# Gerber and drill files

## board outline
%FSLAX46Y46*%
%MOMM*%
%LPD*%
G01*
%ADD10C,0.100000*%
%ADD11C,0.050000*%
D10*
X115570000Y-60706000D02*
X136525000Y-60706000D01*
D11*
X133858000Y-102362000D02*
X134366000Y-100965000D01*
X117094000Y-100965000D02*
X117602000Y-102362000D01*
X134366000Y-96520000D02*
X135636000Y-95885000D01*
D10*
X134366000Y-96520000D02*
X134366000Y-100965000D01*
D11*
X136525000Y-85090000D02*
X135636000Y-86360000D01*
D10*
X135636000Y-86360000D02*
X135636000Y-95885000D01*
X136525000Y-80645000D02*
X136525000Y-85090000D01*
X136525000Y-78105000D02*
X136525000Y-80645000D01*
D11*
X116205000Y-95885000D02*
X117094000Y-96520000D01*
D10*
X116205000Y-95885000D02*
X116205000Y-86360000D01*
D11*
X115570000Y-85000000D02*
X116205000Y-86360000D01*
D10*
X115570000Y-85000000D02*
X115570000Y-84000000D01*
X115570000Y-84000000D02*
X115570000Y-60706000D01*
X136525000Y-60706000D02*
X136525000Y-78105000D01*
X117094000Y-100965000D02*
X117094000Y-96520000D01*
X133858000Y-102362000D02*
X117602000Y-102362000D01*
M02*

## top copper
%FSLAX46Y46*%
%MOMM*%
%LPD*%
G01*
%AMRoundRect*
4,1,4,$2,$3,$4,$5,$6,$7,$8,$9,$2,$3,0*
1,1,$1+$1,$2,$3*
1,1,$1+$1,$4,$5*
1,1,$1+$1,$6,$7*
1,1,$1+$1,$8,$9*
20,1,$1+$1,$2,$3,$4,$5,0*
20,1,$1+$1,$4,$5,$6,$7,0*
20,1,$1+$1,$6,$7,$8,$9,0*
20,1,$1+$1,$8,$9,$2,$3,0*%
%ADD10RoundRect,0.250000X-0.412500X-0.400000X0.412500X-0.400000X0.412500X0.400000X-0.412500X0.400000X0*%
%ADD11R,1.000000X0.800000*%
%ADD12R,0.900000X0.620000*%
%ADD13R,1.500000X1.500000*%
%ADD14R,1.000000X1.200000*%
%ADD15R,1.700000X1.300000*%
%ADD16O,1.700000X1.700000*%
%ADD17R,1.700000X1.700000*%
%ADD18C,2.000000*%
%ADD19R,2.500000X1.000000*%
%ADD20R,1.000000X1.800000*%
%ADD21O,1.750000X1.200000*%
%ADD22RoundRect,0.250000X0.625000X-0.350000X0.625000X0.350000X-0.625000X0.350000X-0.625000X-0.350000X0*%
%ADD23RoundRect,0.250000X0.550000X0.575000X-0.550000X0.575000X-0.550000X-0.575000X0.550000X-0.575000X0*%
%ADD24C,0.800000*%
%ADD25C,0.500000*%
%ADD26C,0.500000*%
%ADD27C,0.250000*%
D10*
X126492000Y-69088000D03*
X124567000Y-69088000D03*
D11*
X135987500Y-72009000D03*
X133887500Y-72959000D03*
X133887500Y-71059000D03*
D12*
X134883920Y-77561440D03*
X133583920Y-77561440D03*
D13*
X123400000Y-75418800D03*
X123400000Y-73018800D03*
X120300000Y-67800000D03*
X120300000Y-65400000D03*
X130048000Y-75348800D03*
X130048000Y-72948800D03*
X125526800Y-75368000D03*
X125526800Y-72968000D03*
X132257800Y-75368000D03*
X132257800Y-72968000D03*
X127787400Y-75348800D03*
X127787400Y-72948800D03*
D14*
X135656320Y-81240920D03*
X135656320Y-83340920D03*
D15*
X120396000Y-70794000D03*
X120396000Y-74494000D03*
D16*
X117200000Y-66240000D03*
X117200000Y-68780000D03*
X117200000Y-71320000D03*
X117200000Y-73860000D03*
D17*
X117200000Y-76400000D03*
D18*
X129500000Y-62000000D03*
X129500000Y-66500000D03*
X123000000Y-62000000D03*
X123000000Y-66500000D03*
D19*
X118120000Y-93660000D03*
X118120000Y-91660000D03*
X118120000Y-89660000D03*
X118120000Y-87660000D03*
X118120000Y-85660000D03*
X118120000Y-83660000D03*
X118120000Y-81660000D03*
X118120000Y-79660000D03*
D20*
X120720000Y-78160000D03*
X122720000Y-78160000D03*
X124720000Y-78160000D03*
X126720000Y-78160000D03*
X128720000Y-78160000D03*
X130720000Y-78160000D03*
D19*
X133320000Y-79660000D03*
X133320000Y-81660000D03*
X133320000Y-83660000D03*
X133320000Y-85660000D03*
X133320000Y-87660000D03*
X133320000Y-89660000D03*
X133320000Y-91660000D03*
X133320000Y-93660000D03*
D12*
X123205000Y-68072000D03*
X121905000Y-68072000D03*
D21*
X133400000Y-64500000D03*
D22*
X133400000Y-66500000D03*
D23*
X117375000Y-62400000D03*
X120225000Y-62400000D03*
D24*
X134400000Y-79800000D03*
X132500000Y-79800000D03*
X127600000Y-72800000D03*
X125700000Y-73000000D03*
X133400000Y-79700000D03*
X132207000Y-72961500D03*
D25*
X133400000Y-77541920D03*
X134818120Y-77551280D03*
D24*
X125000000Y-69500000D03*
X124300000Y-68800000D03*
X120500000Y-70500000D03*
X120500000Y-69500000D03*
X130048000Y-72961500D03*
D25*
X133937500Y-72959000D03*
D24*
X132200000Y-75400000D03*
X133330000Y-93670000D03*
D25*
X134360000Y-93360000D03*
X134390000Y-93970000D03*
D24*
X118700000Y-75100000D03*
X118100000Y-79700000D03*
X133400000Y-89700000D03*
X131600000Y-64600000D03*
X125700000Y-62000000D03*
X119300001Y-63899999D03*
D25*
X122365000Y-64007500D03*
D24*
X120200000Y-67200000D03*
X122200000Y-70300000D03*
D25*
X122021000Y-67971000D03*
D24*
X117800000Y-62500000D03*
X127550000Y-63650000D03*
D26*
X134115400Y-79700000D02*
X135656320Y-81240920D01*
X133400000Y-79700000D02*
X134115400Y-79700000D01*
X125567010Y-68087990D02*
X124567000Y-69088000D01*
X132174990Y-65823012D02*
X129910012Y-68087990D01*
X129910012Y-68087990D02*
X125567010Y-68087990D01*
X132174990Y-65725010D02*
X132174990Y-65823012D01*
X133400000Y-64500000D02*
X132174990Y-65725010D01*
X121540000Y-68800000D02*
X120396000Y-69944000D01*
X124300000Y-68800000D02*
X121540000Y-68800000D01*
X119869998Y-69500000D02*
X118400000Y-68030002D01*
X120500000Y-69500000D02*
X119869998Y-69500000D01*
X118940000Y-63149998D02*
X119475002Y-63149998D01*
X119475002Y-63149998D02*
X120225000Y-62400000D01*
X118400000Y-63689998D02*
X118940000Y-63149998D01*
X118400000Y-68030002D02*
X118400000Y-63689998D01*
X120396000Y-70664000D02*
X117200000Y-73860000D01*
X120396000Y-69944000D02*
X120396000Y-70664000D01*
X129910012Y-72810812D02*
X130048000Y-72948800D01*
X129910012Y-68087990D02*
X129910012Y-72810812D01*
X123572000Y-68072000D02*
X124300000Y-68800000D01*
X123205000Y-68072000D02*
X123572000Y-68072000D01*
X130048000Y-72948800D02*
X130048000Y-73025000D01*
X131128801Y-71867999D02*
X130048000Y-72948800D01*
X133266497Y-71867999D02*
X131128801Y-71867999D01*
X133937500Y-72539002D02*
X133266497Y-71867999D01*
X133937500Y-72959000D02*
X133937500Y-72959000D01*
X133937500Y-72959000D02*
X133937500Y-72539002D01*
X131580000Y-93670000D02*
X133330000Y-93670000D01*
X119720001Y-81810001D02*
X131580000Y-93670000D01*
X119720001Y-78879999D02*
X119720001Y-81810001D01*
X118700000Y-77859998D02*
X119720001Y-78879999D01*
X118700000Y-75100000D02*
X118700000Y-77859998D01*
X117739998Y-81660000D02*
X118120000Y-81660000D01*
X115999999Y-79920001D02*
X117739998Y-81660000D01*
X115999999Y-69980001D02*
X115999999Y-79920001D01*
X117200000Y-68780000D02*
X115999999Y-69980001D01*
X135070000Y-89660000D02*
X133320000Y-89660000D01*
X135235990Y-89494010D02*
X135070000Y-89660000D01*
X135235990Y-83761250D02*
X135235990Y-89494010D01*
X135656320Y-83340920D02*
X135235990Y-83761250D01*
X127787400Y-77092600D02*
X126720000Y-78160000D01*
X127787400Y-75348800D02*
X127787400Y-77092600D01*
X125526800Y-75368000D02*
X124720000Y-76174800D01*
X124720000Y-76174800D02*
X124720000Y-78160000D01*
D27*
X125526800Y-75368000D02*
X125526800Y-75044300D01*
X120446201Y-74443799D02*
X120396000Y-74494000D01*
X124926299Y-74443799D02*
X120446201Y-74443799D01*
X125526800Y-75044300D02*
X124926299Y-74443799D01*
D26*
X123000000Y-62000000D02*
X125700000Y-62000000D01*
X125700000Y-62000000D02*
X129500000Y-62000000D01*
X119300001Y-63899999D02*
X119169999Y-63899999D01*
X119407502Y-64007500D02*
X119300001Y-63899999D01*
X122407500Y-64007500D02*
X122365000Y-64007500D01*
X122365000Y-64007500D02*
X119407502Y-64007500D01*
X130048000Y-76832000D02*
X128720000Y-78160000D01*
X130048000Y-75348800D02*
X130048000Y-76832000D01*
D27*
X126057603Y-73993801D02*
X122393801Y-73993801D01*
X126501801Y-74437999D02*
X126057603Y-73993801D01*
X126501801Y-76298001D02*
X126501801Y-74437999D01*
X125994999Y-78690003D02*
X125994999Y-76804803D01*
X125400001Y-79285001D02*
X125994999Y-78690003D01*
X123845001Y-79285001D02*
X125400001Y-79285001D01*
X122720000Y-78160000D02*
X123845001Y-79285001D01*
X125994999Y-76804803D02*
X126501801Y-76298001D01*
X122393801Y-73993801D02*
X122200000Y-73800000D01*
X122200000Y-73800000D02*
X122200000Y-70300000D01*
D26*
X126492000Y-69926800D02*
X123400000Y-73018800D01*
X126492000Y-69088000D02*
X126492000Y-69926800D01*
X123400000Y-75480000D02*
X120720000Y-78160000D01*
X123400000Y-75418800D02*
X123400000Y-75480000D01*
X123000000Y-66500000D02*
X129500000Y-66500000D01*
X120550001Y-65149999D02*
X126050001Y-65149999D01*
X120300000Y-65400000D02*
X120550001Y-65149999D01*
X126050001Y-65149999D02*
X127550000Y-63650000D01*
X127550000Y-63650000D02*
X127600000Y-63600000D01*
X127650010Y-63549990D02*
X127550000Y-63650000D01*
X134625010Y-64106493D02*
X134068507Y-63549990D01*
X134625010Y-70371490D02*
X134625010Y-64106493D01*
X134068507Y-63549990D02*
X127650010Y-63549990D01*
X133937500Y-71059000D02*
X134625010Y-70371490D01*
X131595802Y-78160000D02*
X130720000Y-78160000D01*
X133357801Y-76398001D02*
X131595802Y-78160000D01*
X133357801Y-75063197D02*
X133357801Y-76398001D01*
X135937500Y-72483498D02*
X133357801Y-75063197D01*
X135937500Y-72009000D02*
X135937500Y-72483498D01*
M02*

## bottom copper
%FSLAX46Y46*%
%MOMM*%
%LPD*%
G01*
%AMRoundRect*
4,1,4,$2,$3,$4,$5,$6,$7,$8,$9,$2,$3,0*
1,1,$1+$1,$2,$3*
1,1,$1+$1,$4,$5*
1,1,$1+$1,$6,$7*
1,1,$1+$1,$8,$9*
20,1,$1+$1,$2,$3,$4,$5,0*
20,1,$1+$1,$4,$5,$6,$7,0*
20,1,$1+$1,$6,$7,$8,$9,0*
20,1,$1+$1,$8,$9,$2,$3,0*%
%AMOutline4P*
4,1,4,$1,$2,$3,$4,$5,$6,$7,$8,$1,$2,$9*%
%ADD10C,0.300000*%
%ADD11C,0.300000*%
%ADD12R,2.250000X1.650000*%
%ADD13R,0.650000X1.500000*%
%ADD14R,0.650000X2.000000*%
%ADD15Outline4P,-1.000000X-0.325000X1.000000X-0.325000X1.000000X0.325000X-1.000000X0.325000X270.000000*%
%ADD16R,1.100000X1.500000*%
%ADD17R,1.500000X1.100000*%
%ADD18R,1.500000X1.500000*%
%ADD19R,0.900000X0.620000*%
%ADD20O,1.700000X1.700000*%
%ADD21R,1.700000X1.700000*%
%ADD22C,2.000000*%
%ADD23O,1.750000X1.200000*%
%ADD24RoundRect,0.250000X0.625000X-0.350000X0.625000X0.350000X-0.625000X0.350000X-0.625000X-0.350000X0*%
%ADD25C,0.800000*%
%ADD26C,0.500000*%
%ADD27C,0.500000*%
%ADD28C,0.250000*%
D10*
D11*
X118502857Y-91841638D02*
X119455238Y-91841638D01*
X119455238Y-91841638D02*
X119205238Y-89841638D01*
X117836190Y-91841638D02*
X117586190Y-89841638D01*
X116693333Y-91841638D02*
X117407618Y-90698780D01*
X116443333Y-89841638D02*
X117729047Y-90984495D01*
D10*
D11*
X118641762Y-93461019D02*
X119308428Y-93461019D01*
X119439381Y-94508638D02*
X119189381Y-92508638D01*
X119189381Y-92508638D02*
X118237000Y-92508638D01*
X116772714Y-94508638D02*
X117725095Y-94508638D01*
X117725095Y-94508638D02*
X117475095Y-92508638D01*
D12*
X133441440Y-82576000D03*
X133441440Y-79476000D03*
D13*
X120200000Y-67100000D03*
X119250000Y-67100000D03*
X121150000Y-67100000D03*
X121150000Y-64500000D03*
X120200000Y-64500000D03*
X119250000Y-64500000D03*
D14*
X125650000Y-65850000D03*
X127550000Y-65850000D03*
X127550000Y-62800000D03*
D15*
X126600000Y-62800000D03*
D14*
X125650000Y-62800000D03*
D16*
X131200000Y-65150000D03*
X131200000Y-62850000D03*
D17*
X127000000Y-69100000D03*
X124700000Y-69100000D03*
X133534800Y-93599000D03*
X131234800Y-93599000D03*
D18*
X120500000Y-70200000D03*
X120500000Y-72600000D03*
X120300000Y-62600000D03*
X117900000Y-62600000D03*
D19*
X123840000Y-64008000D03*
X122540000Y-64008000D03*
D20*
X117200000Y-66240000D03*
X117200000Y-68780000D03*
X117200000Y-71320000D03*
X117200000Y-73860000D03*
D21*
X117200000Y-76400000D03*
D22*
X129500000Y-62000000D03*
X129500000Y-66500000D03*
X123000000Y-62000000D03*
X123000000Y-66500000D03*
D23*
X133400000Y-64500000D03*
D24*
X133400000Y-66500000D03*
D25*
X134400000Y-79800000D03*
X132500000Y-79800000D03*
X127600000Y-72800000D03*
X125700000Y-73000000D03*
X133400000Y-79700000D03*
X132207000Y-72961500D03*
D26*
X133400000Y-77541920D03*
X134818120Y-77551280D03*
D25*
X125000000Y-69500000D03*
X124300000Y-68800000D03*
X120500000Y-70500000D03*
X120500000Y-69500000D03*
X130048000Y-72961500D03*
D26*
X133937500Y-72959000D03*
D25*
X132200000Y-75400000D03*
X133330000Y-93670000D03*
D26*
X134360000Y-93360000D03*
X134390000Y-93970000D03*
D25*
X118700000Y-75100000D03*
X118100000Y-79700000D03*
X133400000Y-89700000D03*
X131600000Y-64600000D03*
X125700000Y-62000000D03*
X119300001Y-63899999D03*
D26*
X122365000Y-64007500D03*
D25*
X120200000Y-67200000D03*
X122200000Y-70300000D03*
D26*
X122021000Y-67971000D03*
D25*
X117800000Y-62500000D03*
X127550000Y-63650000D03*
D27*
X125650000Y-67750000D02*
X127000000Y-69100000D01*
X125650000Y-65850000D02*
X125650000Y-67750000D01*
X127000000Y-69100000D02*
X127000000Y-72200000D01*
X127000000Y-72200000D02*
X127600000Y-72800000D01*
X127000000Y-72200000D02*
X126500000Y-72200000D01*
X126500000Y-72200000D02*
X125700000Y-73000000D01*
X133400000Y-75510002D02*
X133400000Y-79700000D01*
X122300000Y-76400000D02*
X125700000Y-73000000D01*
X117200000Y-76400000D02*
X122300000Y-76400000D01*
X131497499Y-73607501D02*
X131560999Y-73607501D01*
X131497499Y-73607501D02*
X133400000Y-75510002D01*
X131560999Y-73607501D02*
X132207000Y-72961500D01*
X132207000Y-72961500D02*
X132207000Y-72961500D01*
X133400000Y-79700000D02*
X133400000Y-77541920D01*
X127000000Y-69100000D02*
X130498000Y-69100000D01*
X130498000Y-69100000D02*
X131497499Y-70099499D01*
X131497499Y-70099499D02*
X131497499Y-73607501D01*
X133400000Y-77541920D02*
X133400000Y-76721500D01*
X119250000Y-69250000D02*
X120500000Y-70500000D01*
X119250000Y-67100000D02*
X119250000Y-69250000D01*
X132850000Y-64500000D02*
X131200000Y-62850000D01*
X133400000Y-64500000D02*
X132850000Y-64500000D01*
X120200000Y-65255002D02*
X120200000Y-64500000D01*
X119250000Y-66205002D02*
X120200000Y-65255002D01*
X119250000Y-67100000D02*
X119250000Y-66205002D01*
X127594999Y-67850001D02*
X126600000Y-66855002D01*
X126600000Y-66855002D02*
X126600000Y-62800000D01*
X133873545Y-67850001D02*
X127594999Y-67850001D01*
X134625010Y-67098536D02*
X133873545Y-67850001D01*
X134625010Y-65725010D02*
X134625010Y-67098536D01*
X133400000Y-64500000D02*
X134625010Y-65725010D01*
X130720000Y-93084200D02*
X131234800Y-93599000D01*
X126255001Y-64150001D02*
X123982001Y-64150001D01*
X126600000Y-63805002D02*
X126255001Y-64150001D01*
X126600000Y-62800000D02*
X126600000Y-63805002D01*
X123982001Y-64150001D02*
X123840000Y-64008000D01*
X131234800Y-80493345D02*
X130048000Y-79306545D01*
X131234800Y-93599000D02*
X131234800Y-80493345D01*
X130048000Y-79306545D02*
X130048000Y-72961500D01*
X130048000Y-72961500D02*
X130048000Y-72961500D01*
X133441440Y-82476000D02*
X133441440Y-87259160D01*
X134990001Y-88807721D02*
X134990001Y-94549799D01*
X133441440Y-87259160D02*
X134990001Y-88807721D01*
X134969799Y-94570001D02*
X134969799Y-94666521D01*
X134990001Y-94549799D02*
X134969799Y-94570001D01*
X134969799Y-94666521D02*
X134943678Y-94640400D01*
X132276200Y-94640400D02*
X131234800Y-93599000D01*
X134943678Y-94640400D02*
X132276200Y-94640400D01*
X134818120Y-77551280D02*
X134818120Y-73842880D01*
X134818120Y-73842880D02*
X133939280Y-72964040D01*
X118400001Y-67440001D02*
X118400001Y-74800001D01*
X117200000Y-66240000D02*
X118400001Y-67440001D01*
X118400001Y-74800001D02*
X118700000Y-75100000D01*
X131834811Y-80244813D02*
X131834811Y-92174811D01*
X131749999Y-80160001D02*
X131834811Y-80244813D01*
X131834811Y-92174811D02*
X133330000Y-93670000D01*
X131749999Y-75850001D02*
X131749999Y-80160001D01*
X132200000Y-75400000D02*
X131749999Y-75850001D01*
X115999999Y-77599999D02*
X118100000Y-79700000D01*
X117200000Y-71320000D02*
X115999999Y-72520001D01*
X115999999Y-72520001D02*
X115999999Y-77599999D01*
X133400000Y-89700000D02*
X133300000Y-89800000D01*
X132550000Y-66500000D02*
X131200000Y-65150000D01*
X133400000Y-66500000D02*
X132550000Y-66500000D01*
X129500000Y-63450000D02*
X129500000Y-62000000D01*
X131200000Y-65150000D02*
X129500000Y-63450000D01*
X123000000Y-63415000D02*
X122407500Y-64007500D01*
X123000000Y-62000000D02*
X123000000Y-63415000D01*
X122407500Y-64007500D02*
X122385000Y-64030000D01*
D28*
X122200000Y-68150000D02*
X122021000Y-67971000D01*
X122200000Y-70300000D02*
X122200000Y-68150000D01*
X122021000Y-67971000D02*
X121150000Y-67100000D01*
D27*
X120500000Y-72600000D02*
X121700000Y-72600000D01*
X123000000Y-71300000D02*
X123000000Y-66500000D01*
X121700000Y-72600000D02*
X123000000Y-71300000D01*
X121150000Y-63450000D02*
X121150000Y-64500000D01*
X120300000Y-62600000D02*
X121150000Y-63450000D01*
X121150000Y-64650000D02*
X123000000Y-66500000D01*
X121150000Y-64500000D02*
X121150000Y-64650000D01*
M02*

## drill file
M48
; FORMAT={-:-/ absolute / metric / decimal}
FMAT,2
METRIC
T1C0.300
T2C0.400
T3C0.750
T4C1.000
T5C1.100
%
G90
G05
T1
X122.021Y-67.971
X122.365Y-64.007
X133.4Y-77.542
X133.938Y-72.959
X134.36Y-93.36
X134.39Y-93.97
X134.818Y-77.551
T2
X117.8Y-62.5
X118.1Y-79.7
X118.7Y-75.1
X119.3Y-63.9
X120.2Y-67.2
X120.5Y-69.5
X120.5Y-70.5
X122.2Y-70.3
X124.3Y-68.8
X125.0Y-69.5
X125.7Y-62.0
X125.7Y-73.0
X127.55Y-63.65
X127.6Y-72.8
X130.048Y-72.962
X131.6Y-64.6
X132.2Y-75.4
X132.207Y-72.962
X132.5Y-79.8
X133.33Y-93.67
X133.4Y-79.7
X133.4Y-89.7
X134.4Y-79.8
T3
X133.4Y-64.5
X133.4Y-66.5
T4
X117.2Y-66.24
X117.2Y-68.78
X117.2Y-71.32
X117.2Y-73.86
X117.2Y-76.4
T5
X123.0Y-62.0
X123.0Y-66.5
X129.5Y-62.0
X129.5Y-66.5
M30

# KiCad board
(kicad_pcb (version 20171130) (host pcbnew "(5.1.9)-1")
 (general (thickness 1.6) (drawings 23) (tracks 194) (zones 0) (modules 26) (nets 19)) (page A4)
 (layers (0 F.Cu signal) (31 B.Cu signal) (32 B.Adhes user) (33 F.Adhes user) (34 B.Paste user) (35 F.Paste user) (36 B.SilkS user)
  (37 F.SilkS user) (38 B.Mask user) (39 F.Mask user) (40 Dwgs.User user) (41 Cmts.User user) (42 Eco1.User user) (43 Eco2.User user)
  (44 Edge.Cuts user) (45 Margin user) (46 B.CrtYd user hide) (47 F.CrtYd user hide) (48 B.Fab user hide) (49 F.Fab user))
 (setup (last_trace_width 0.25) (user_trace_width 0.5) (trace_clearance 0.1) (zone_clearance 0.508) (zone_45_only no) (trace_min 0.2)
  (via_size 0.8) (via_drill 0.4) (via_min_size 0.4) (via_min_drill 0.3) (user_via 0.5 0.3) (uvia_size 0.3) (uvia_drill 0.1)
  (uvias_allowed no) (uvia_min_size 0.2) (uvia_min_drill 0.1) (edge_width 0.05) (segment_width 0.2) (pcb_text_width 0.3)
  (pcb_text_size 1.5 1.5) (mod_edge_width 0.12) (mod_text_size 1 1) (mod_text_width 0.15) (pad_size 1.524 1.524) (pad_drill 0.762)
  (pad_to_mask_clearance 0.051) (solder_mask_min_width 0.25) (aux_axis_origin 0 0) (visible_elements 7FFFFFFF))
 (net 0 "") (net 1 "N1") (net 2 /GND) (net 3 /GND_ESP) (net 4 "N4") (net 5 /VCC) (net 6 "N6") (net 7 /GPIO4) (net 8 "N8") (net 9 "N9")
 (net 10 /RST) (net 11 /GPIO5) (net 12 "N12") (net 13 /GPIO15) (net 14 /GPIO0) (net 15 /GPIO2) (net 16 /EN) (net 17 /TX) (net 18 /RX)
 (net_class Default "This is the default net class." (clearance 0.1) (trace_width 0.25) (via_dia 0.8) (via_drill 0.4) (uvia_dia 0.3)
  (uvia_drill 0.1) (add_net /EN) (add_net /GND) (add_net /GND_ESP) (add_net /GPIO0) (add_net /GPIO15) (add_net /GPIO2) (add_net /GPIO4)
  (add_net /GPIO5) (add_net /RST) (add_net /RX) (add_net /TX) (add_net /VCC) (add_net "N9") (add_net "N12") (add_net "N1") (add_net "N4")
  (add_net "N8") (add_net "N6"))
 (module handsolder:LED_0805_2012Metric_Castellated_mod (layer F.Cu) (at 125.5295 69.088)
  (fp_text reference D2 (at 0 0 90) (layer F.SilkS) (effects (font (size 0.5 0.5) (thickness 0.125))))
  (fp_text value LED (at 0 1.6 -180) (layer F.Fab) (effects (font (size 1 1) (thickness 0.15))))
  (pad 2 smd roundrect (at 0.9625 0) (size 1.325 1.3) (layers F.Cu F.Paste F.Mask) (roundrect_rratio 0.1923076923076923) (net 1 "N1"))
  (pad 1 smd roundrect (at -0.9625 0) (size 1.325 1.3) (layers F.Cu F.Paste F.Mask) (roundrect_rratio 0.1923076923076923) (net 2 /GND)))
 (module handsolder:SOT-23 (layer F.Cu) (at 134.9375 72.009)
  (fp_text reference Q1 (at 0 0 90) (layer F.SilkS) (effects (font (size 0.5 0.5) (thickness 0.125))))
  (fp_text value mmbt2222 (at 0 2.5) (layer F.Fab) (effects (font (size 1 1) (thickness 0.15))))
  (pad 3 smd rect (at 1.05 0) (size 1 0.8) (layers F.Cu F.Paste F.Mask) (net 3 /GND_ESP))
  (pad 2 smd rect (at -1.05 0.95) (size 1 0.8) (layers F.Cu F.Paste F.Mask) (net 2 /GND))
  (pad 1 smd rect (at -1.05 -0.95) (size 1 0.8) (layers F.Cu F.Paste F.Mask) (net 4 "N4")))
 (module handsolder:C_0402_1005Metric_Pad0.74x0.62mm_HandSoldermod (layer F.Cu) (at 134.23392 77.56144)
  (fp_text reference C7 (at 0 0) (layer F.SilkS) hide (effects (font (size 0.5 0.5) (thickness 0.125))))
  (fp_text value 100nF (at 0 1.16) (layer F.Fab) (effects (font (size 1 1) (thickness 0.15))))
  (pad 2 smd rect (at 0.65 0) (size 0.9 0.62) (layers F.Cu F.Paste F.Mask) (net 2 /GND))
  (pad 1 smd rect (at -0.65 0) (size 0.9 0.62) (layers F.Cu F.Paste F.Mask) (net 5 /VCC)))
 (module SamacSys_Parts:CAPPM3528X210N (layer B.Cu) (at 133.44144 81.026 270)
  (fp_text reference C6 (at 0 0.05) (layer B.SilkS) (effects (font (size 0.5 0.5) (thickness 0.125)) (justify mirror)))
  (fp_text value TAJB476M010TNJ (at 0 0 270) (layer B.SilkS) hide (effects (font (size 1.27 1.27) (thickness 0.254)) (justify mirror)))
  (pad 2 smd rect (at 1.55 0 270) (size 1.65 2.25) (layers B.Cu B.Paste B.Mask) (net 2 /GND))
  (pad 1 smd rect (at -1.55 0 270) (size 1.65 2.25) (layers B.Cu B.Paste B.Mask) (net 5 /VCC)))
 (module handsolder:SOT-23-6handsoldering (layer B.Cu) (at 120.2 65.8 270)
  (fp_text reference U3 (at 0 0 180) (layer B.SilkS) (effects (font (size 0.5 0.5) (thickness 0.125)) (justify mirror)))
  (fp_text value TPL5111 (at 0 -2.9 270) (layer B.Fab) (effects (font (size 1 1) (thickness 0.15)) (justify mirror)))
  (pad 5 smd rect (at 1.3 0 270) (size 1.5 0.65) (layers B.Cu B.Paste B.Mask) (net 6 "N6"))
  (pad 6 smd rect (at 1.3 0.95 270) (size 1.5 0.65) (layers B.Cu B.Paste B.Mask) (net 2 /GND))
  (pad 4 smd rect (at 1.3 -0.95 270) (size 1.5 0.65) (layers B.Cu B.Paste B.Mask) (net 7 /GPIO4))
  (pad 3 smd rect (at -1.3 -0.95 270) (size 1.5 0.65) (layers B.Cu B.Paste B.Mask) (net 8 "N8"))
  (pad 2 smd rect (at -1.3 0 270) (size 1.5 0.65) (layers B.Cu B.Paste B.Mask) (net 2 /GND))
  (pad 1 smd rect (at -1.3 0.95 270) (size 1.5 0.65) (layers B.Cu B.Paste B.Mask) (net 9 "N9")))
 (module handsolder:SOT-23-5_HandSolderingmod (layer B.Cu) (at 126.6 64.35 270)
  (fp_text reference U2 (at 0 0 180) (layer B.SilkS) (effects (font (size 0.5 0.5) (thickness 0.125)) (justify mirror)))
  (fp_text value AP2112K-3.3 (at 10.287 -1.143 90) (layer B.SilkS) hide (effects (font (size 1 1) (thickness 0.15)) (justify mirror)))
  (pad 5 smd rect (at 1.5 0.95 270) (size 2 0.65) (layers B.Cu B.Paste B.Mask) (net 5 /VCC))
  (pad 4 smd rect (at 1.5 -0.95 270) (size 2 0.65) (layers B.Cu B.Paste B.Mask))
  (pad 3 smd rect (at -1.55 -0.95 270) (size 2 0.65) (layers B.Cu B.Paste B.Mask) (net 4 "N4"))
  (pad 2 smd trapezoid (at -1.55 0 270) (size 2 0.65) (layers B.Cu B.Paste B.Mask) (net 2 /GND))
  (pad 1 smd rect (at -1.55 0.95 270) (size 2 0.65) (layers B.Cu B.Paste B.Mask) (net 9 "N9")))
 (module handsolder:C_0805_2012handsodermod (layer B.Cu) (at 131.2 64 270)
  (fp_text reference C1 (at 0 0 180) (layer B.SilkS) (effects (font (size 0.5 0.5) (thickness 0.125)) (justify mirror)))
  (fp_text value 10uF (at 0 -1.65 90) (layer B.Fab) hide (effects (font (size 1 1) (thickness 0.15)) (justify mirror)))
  (pad 2 smd rect (at 1.15 0 270) (size 1.5 1.1) (layers B.Cu B.Paste B.Mask) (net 9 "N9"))
  (pad 1 smd rect (at -1.15 0 270) (size 1.5 1.1) (layers B.Cu B.Paste B.Mask) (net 2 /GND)))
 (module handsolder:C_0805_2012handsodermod (layer B.Cu) (at 125.85 69.1)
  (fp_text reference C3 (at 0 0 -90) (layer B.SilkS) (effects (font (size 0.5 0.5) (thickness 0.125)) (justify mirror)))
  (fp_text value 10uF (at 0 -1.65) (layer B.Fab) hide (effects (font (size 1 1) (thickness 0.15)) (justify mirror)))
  (pad 2 smd rect (at 1.15 0) (size 1.5 1.1) (layers B.Cu B.Paste B.Mask) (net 5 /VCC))
  (pad 1 smd rect (at -1.15 0) (size 1.5 1.1) (layers B.Cu B.Paste B.Mask) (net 2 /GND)))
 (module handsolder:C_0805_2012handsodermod (layer B.Cu) (at 132.3848 93.599)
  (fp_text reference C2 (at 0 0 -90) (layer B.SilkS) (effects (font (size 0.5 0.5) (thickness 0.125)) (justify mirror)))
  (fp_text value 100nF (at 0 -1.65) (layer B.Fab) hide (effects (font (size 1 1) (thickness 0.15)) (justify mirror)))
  (pad 2 smd rect (at 1.15 0) (size 1.5 1.1) (layers B.Cu B.Paste B.Mask) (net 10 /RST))
  (pad 1 smd rect (at -1.15 0) (size 1.5 1.1) (layers B.Cu B.Paste B.Mask) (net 2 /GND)))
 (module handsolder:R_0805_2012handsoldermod (layer B.Cu) (at 120.5 71.4 90)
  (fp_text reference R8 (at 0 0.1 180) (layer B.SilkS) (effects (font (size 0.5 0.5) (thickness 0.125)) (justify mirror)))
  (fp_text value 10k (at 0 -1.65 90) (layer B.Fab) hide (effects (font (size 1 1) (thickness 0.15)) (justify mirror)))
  (pad 2 smd rect (at 1.2 0 90) (size 1.5 1.5) (layers B.Cu B.Paste B.Mask) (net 2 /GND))
  (pad 1 smd rect (at -1.2 0 90) (size 1.5 1.5) (layers B.Cu B.Paste B.Mask) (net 8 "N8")))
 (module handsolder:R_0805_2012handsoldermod (layer F.Cu) (at 123.4 74.2188 270)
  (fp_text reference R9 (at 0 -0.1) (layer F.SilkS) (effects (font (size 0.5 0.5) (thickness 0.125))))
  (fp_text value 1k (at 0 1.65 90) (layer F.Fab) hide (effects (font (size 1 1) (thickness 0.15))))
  (pad 2 smd rect (at 1.2 0 270) (size 1.5 1.5) (layers F.Cu F.Paste F.Mask) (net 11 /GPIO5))
  (pad 1 smd rect (at -1.2 0 270) (size 1.5 1.5) (layers F.Cu F.Paste F.Mask) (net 1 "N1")))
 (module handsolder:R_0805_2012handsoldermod (layer F.Cu) (at 120.3 66.6 270)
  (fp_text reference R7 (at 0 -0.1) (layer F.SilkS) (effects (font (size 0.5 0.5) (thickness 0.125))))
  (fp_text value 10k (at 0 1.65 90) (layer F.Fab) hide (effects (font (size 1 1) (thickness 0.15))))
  (pad 2 smd rect (at 1.2 0 270) (size 1.5 1.5) (layers F.Cu F.Paste F.Mask) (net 6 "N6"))
  (pad 1 smd rect (at -1.2 0 270) (size 1.5 1.5) (layers F.Cu F.Paste F.Mask) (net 4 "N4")))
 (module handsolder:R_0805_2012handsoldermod (layer B.Cu) (at 119.1 62.6)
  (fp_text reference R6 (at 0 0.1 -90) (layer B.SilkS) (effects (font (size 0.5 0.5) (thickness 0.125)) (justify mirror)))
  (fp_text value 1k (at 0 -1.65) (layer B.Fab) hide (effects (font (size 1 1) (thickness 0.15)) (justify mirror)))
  (pad 2 smd rect (at 1.2 0) (size 1.5 1.5) (layers B.Cu B.Paste B.Mask) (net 8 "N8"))
  (pad 1 smd rect (at -1.2 0) (size 1.5 1.5) (layers B.Cu B.Paste B.Mask) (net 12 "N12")))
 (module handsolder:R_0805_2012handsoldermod (layer F.Cu) (at 130.048 74.1488 270)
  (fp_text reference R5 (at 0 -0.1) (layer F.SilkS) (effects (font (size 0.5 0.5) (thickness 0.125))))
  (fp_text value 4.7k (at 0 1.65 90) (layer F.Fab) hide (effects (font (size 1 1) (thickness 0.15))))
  (pad 2 smd rect (at 1.2 0 270) (size 1.5 1.5) (layers F.Cu F.Paste F.Mask) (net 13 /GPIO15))
  (pad 1 smd rect (at -1.2 0 270) (size 1.5 1.5) (layers F.Cu F.Paste F.Mask) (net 2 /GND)))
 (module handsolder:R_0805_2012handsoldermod (layer F.Cu) (at 125.5268 74.168 270)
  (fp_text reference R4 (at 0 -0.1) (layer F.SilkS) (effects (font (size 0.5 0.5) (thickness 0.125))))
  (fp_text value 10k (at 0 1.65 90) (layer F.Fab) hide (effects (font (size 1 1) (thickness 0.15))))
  (pad 2 smd rect (at 1.2 0 270) (size 1.5 1.5) (layers F.Cu F.Paste F.Mask) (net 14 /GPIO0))
  (pad 1 smd rect (at -1.2 0 270) (size 1.5 1.5) (layers F.Cu F.Paste F.Mask) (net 5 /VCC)))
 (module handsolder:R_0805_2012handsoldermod (layer F.Cu) (at 132.2578 74.168 270)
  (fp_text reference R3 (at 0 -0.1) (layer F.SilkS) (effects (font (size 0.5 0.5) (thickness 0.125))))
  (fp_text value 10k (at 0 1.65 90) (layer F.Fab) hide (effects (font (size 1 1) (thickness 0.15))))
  (pad 2 smd rect (at 1.2 0 270) (size 1.5 1.5) (layers F.Cu F.Paste F.Mask) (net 10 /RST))
  (pad 1 smd rect (at -1.2 0 270) (size 1.5 1.5) (layers F.Cu F.Paste F.Mask) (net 5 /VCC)))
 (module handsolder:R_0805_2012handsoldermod (layer F.Cu) (at 127.7874 74.1488 270)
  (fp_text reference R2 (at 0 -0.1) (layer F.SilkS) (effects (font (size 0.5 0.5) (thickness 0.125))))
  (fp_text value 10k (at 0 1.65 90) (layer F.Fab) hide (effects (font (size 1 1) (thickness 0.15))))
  (pad 2 smd rect (at 1.2 0 270) (size 1.5 1.5) (layers F.Cu F.Paste F.Mask) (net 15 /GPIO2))
  (pad 1 smd rect (at -1.2 0 270) (size 1.5 1.5) (layers F.Cu F.Paste F.Mask) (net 5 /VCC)))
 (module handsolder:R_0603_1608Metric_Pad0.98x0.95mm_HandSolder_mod (layer F.Cu) (at 135.65632 82.29092 90)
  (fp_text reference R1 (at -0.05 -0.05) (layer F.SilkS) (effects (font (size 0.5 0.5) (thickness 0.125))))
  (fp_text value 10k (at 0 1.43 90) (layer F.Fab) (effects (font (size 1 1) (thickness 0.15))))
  (pad 2 smd rect (at 1.05 0 90) (size 1.2 1) (layers F.Cu F.Paste F.Mask) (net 5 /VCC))
  (pad 1 smd rect (at -1.05 0 90) (size 1.2 1) (layers F.Cu F.Paste F.Mask) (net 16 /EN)))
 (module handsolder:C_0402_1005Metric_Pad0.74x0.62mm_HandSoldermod (layer B.Cu) (at 123.19 64.008)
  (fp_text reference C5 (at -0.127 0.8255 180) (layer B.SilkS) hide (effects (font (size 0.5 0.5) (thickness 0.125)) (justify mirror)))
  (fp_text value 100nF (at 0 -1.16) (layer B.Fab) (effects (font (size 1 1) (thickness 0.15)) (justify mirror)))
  (pad 2 smd rect (at 0.65 0) (size 0.9 0.62) (layers B.Cu B.Paste B.Mask) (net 2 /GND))
  (pad 1 smd rect (at -0.65 0) (size 0.9 0.62) (layers B.Cu B.Paste B.Mask) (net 9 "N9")))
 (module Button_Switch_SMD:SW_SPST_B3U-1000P (layer F.Cu) (at 120.396 72.644 90)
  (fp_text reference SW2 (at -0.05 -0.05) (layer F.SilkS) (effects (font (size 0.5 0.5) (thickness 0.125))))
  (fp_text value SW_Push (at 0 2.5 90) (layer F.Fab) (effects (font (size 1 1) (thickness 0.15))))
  (pad 2 smd rect (at 1.85 0 90) (size 1.3 1.7) (layers F.Cu F.Paste F.Mask) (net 2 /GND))
  (pad 1 smd rect (at -1.85 0 90) (size 1.3 1.7) (layers F.Cu F.Paste F.Mask) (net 14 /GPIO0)))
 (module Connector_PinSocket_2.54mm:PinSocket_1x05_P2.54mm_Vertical (layer F.Cu) (at 117.2 76.4 180)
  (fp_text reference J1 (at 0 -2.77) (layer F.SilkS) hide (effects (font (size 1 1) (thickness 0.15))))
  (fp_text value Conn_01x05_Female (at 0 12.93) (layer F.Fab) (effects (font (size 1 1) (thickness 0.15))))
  (pad 5 thru_hole oval (at 0 10.16 180) (size 1.7 1.7) (drill 1) (layers *.Cu *.Mask) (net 10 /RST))
  (pad 4 thru_hole oval (at 0 7.62 180) (size 1.7 1.7) (drill 1) (layers *.Cu *.Mask) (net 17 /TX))
  (pad 3 thru_hole oval (at 0 5.08 180) (size 1.7 1.7) (drill 1) (layers *.Cu *.Mask) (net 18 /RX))
  (pad 2 thru_hole oval (at 0 2.54 180) (size 1.7 1.7) (drill 1) (layers *.Cu *.Mask) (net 2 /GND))
  (pad 1 thru_hole rect (at 0 0 180) (size 1.7 1.7) (drill 1) (layers *.Cu *.Mask) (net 5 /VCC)))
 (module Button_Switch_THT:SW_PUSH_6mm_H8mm (layer F.Cu) (at 123 62)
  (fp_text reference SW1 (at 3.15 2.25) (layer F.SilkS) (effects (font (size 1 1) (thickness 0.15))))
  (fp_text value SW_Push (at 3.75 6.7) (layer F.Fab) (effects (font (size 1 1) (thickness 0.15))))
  (pad 1 thru_hole circle (at 6.5 0 90) (size 2 2) (drill 1.1) (layers *.Cu *.Mask) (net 9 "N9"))
  (pad 2 thru_hole circle (at 6.5 4.5 90) (size 2 2) (drill 1.1) (layers *.Cu *.Mask) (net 8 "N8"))
  (pad 1 thru_hole circle (at 0 0 90) (size 2 2) (drill 1.1) (layers *.Cu *.Mask) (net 9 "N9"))
  (pad 2 thru_hole circle (at 0 4.5 90) (size 2 2) (drill 1.1) (layers *.Cu *.Mask) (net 8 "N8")))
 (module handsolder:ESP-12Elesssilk (layer F.Cu) (at 125.72 90.16 180)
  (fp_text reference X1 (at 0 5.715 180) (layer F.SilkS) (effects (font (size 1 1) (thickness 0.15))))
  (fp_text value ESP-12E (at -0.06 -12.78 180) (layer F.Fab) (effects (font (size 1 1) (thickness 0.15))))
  (pad 22 smd rect (at 7.6 -3.5 180) (size 2.5 1) (layers F.Cu F.Paste F.Mask))
  (pad 21 smd rect (at 7.6 -1.5 180) (size 2.5 1) (layers F.Cu F.Paste F.Mask))
  (pad 20 smd rect (at 7.6 0.5 180) (size 2.5 1) (layers F.Cu F.Paste F.Mask))
  (pad 19 smd rect (at 7.6 2.5 180) (size 2.5 1) (layers F.Cu F.Paste F.Mask))
  (pad 18 smd rect (at 7.6 4.5 180) (size 2.5 1) (layers F.Cu F.Paste F.Mask))
  (pad 17 smd rect (at 7.6 6.5 180) (size 2.5 1) (layers F.Cu F.Paste F.Mask))
  (pad 16 smd rect (at 7.6 8.5 180) (size 2.5 1) (layers F.Cu F.Paste F.Mask) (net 17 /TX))
  (pad 15 smd rect (at 7.6 10.5 180) (size 2.5 1) (layers F.Cu F.Paste F.Mask) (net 18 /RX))
  (pad 14 smd rect (at 5 12 180) (size 1 1.8) (layers F.Cu F.Paste F.Mask) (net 11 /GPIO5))
  (pad 13 smd rect (at 3 12 180) (size 1 1.8) (layers F.Cu F.Paste F.Mask) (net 7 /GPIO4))
  (pad 12 smd rect (at 1 12 180) (size 1 1.8) (layers F.Cu F.Paste F.Mask) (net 14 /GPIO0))
  (pad 11 smd rect (at -1 12 180) (size 1 1.8) (layers F.Cu F.Paste F.Mask) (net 15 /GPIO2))
  (pad 10 smd rect (at -3 12 180) (size 1 1.8) (layers F.Cu F.Paste F.Mask) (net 13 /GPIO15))
  (pad 9 smd rect (at -5 12 180) (size 1 1.8) (layers F.Cu F.Paste F.Mask) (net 3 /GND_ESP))
  (pad 8 smd rect (at -7.6 10.5 180) (size 2.5 1) (layers F.Cu F.Paste F.Mask) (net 5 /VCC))
  (pad 7 smd rect (at -7.6 8.5 180) (size 2.5 1) (layers F.Cu F.Paste F.Mask))
  (pad 6 smd rect (at -7.6 6.5 180) (size 2.5 1) (layers F.Cu F.Paste F.Mask))
  (pad 5 smd rect (at -7.6 4.5 180) (size 2.5 1) (layers F.Cu F.Paste F.Mask))
  (pad 4 smd rect (at -7.6 2.5 180) (size 2.5 1) (layers F.Cu F.Paste F.Mask))
  (pad 3 smd rect (at -7.6 0.5 180) (size 2.5 1) (layers F.Cu F.Paste F.Mask) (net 16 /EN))
  (pad 2 smd rect (at -7.6 -1.5 180) (size 2.5 1) (layers F.Cu F.Paste F.Mask))
  (pad 1 smd rect (at -7.6 -3.5 180) (size 2.5 1) (layers F.Cu F.Paste F.Mask) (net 10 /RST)))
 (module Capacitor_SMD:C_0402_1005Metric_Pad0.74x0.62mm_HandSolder (layer F.Cu) (at 122.555 68.072)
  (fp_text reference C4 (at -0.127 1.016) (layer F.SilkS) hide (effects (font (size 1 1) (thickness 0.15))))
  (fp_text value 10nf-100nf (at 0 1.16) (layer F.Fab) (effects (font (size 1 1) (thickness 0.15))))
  (pad 2 smd rect (at 0.65 0) (size 0.9 0.62) (layers F.Cu F.Paste F.Mask) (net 2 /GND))
  (pad 1 smd rect (at -0.65 0) (size 0.9 0.62) (layers F.Cu F.Paste F.Mask) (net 7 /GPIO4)))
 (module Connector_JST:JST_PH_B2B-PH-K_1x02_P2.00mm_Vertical (layer F.Cu) (at 133.4 66.5 90)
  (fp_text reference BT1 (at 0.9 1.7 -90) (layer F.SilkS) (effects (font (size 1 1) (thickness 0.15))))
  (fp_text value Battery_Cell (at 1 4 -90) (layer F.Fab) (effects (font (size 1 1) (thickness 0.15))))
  (pad 2 thru_hole oval (at 2 0 90) (size 1.2 1.75) (drill 0.75) (layers *.Cu *.Mask) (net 2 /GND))
  (pad 1 thru_hole roundrect (at 0 0 90) (size 1.2 1.75) (drill 0.75) (layers *.Cu *.Mask) (roundrect_rratio 0.208333) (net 9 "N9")))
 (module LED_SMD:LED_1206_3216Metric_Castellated (layer F.Cu) (at 118.8 62.4 180)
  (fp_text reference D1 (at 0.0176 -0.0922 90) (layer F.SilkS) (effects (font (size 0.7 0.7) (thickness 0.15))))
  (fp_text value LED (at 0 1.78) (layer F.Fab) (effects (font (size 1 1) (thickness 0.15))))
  (pad 2 smd roundrect (at 1.425 0 180) (size 1.6 1.65) (layers F.Cu F.Paste F.Mask) (roundrect_rratio 0.15625) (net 12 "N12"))
  (pad 1 smd roundrect (at -1.425 0 180) (size 1.6 1.65) (layers F.Cu F.Paste F.Mask) (roundrect_rratio 0.15625) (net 2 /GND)))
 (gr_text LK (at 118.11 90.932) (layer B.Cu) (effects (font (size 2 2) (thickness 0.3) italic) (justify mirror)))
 (gr_line (start 115.57 60.706) (end 136.525 60.706) (layer Edge.Cuts) (width 0.1))
 (gr_line (start 133.858 102.362) (end 134.366 100.965) (layer Edge.Cuts) (width 0.05))
 (gr_line (start 117.094 100.965) (end 117.602 102.362) (layer Edge.Cuts) (width 0.05))
 (gr_line (start 134.366 96.52) (end 135.636 95.885) (layer Edge.Cuts) (width 0.05))
 (gr_line (start 134.366 96.52) (end 134.366 100.965) (layer Edge.Cuts) (width 0.1))
 (gr_line (start 136.525 85.09) (end 135.636 86.36) (layer Edge.Cuts) (width 0.05))
 (gr_line (start 135.636 86.36) (end 135.636 95.885) (layer Edge.Cuts) (width 0.1))
 (gr_line (start 136.525 80.645) (end 136.525 85.09) (layer Edge.Cuts) (width 0.1))
 (gr_line (start 136.525 78.105) (end 136.525 80.645) (layer Edge.Cuts) (width 0.1))
 (gr_line (start 116.205 95.885) (end 117.094 96.52) (layer Edge.Cuts) (width 0.05))
 (gr_line (start 116.205 95.885) (end 116.205 86.36) (layer Edge.Cuts) (width 0.1))
 (gr_line (start 115.57 85) (end 116.205 86.36) (layer Edge.Cuts) (width 0.05))
 (gr_line (start 115.57 85) (end 115.57 84) (layer Edge.Cuts) (width 0.1))
 (gr_line (start 115.57 84) (end 115.57 60.706) (layer Edge.Cuts) (width 0.1))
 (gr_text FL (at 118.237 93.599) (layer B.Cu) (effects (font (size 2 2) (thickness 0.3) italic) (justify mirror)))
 (gr_line (start 136.525 60.706) (end 136.525 78.105) (layer Edge.Cuts) (width 0.1))
 (gr_line (start 117.094 100.965) (end 117.094 96.52) (layer Edge.Cuts) (width 0.1))
 (gr_line (start 133.858 102.362) (end 117.602 102.362) (layer Edge.Cuts) (width 0.1))
 (via (at 134.4 79.8) (size 0.8) (drill 0.4) (layers F.Cu B.Cu) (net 5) (status 30))
 (via (at 132.5 79.8) (size 0.8) (drill 0.4) (layers F.Cu B.Cu) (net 5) (status 30))
 (segment (start 125.65 67.75) (end 127 69.1) (width 0.5) (layer B.Cu) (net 5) (status 20))
 (segment (start 125.65 65.85) (end 125.65 67.75) (width 0.5) (layer B.Cu) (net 5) (status 10))
 (segment (start 127 69.1) (end 127 72.2) (width 0.5) (layer B.Cu) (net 5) (status 10))
 (segment (start 127 72.2) (end 127.6 72.8) (width 0.5) (layer B.Cu) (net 5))
 (segment (start 127 72.2) (end 126.5 72.2) (width 0.5) (layer B.Cu) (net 5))
 (segment (start 126.5 72.2) (end 125.7 73) (width 0.5) (layer B.Cu) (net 5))
 (via (at 127.6 72.8) (size 0.8) (drill 0.4) (layers F.Cu B.Cu) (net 5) (status 30))
 (via (at 125.7 73) (size 0.8) (drill 0.4) (layers F.Cu B.Cu) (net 5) (status 30))
 (segment (start 133.4 75.510002) (end 133.4 79.7) (width 0.5) (layer B.Cu) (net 5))
 (via (at 133.4 79.7) (size 0.8) (drill 0.4) (layers F.Cu B.Cu) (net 5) (status 30))
 (segment (start 122.3 76.4) (end 125.7 73) (width 0.5) (layer B.Cu) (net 5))
 (segment (start 117.2 76.4) (end 122.3 76.4) (width 0.5) (layer B.Cu) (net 5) (status 10))
 (segment (start 131.497499 73.607501) (end 131.560999 73.607501) (width 0.5) (layer B.Cu) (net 5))
 (segment (start 131.497499 73.607501) (end 133.4 75.510002) (width 0.5) (layer B.Cu) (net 5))
 (segment (start 131.560999 73.607501) (end 132.207 72.9615) (width 0.5) (layer B.Cu) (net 5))
 (segment (start 132.207 72.9615) (end 132.207 72.9615) (width 0.5) (layer B.Cu) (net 5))
 (via (at 132.207 72.9615) (size 0.8) (drill 0.4) (layers F.Cu B.Cu) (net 5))
 (segment (start 133.4 79.7) (end 133.4 77.54192) (width 0.5) (layer B.Cu) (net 5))
 (segment (start 127 69.1) (end 130.498 69.1) (width 0.5) (layer B.Cu) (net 5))
 (segment (start 130.498 69.1) (end 131.497499 70.099499) (width 0.5) (layer B.Cu) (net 5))
 (segment (start 131.497499 70.099499) (end 131.497499 73.607501) (width 0.5) (layer B.Cu) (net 5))
 (segment (start 134.1154 79.7) (end 135.65632 81.24092) (width 0.5) (layer F.Cu) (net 5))
 (segment (start 133.4 79.7) (end 134.1154 79.7) (width 0.5) (layer F.Cu) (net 5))
 (segment (start 133.4 77.54192) (end 133.4 76.7215) (width 0.5) (layer B.Cu) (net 5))
 (via (at 133.4 77.54192) (size 0.5) (drill 0.3) (layers F.Cu B.Cu) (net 5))
 (via (at 134.81812 77.55128) (size 0.5) (drill 0.3) (layers F.Cu B.Cu) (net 2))
 (via (at 125 69.5) (size 0.8) (drill 0.4) (layers F.Cu B.Cu) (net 2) (status 30))
 (via (at 124.3 68.8) (size 0.8) (drill 0.4) (layers F.Cu B.Cu) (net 2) (status 30))
 (via (at 120.5 70.5) (size 0.8) (drill 0.4) (layers F.Cu B.Cu) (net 2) (status 30))
 (via (at 120.5 69.5) (size 0.8) (drill 0.4) (layers F.Cu B.Cu) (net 2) (status 30))
 (segment (start 119.25 69.25) (end 120.5 70.5) (width 0.5) (layer B.Cu) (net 2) (status 20))
 (segment (start 119.25 67.1) (end 119.25 69.25) (width 0.5) (layer B.Cu) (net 2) (status 10))
 (segment (start 132.85 64.5) (end 131.2 62.85) (width 0.5) (layer B.Cu) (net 2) (status 30))
 (segment (start 133.4 64.5) (end 132.85 64.5) (width 0.5) (layer B.Cu) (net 2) (status 30))
 (segment (start 120.2 65.255002) (end 120.2 64.5) (width 0.5) (layer B.Cu) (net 2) (status 20))
 (segment (start 119.25 66.205002) (end 120.2 65.255002) (width 0.5) (layer B.Cu) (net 2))
 (segment (start 119.25 67.1) (end 119.25 66.205002) (width 0.5) (layer B.Cu) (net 2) (status 10))
 (segment (start 127.594999 67.850001) (end 126.6 66.855002) (width 0.5) (layer B.Cu) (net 2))
 (segment (start 126.6 66.855002) (end 126.6 62.8) (width 0.5) (layer B.Cu) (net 2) (status 20))
 (segment (start 133.873545 67.850001) (end 127.594999 67.850001) (width 0.5) (layer B.Cu) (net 2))
 (segment (start 134.62501 67.098536) (end 133.873545 67.850001) (width 0.5) (layer B.Cu) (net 2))
 (segment (start 134.62501 65.72501) (end 134.62501 67.098536) (width 0.5) (layer B.Cu) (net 2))
 (segment (start 133.4 64.5) (end 134.62501 65.72501) (width 0.5) (layer B.Cu) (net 2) (status 10))
 (segment (start 125.56701 68.08799) (end 124.567 69.088) (width 0.5) (layer F.Cu) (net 2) (status 20))
 (segment (start 132.17499 65.823012) (end 129.910012 68.08799) (width 0.5) (layer F.Cu) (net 2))
 (segment (start 129.910012 68.08799) (end 125.56701 68.08799) (width 0.5) (layer F.Cu) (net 2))
 (segment (start 132.17499 65.72501) (end 132.17499 65.823012) (width 0.5) (layer F.Cu) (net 2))
 (segment (start 133.4 64.5) (end 132.17499 65.72501) (width 0.5) (layer F.Cu) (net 2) (status 10))
 (segment (start 121.54 68.8) (end 120.396 69.944) (width 0.5) (layer F.Cu) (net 2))
 (segment (start 124.3 68.8) (end 121.54 68.8) (width 0.5) (layer F.Cu) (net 2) (status 10))
 (segment (start 119.869998 69.5) (end 118.4 68.030002) (width 0.5) (layer F.Cu) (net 2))
 (segment (start 120.5 69.5) (end 119.869998 69.5) (width 0.5) (layer F.Cu) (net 2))
 (segment (start 118.94 63.149998) (end 119.475002 63.149998) (width 0.5) (layer F.Cu) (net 2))
 (segment (start 119.475002 63.149998) (end 120.225 62.4) (width 0.5) (layer F.Cu) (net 2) (status 20))
 (segment (start 118.4 63.689998) (end 118.94 63.149998) (width 0.5) (layer F.Cu) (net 2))
 (segment (start 118.4 68.030002) (end 118.4 63.689998) (width 0.5) (layer F.Cu) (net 2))
 (segment (start 120.396 70.664) (end 117.2 73.86) (width 0.5) (layer F.Cu) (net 2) (status 30))
 (segment (start 120.396 69.944) (end 120.396 70.664) (width 0.5) (layer F.Cu) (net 2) (status 20))
 (segment (start 129.910012 72.810812) (end 130.048 72.9488) (width 0.5) (layer F.Cu) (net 2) (status 30))
 (segment (start 129.910012 68.08799) (end 129.910012 72.810812) (width 0.5) (layer F.Cu) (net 2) (status 20))
 (segment (start 130.72 93.0842) (end 131.2348 93.599) (width 0.5) (layer B.Cu) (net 2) (status 30))
 (segment (start 123.572 68.072) (end 124.3 68.8) (width 0.5) (layer F.Cu) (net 2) (status 30))
 (segment (start 123.205 68.072) (end 123.572 68.072) (width 0.5) (layer F.Cu) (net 2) (status 30))
 (segment (start 126.255001 64.150001) (end 123.982001 64.150001) (width 0.5) (layer B.Cu) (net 2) (status 20))
 (segment (start 126.6 63.805002) (end 126.255001 64.150001) (width 0.5) (layer B.Cu) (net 2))
 (segment (start 126.6 62.8) (end 126.6 63.805002) (width 0.5) (layer B.Cu) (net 2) (status 10))
 (segment (start 123.982001 64.150001) (end 123.84 64.008) (width 0.5) (layer B.Cu) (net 2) (status 30))
 (segment (start 130.048 72.9488) (end 130.048 73.025) (width 0.5) (layer F.Cu) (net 2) (status 30))
 (segment (start 131.128801 71.867999) (end 130.048 72.9488) (width 0.5) (layer F.Cu) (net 2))
 (segment (start 133.266497 71.867999) (end 131.128801 71.867999) (width 0.5) (layer F.Cu) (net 2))
 (segment (start 133.9375 72.539002) (end 133.266497 71.867999) (width 0.5) (layer F.Cu) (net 2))
 (segment (start 133.9375 72.959) (end 133.9375 72.959) (width 0.5) (layer F.Cu) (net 2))
 (segment (start 131.2348 80.493345) (end 130.048 79.306545) (width 0.5) (layer B.Cu) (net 2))
 (segment (start 131.2348 93.599) (end 131.2348 80.493345) (width 0.5) (layer B.Cu) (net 2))
 (segment (start 130.048 79.306545) (end 130.048 72.9615) (width 0.5) (layer B.Cu) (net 2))
 (segment (start 130.048 72.9615) (end 130.048 72.9615) (width 0.5) (layer B.Cu) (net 2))
 (via (at 130.048 72.9615) (size 0.8) (drill 0.4) (layers F.Cu B.Cu) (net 2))
 (segment (start 133.44144 82.476) (end 133.44144 87.25916) (width 0.5) (layer B.Cu) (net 2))
 (segment (start 134.990001 88.807721) (end 134.990001 94.549799) (width 0.5) (layer B.Cu) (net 2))
 (segment (start 133.44144 87.25916) (end 134.990001 88.807721) (width 0.5) (layer B.Cu) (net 2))
 (segment (start 134.969799 94.570001) (end 134.969799 94.666521) (width 0.5) (layer B.Cu) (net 2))
 (segment (start 134.990001 94.549799) (end 134.969799 94.570001) (width 0.5) (layer B.Cu) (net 2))
 (segment (start 134.969799 94.666521) (end 134.943678 94.6404) (width 0.5) (layer B.Cu) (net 2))
 (segment (start 132.2762 94.6404) (end 131.2348 93.599) (width 0.5) (layer B.Cu) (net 2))
 (segment (start 134.943678 94.6404) (end 132.2762 94.6404) (width 0.5) (layer B.Cu) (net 2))
 (segment (start 134.81812 77.55128) (end 134.81812 73.84288) (width 0.5) (layer B.Cu) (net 2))
 (segment (start 134.81812 73.84288) (end 133.93928 72.96404) (width 0.5) (layer B.Cu) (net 2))
 (segment (start 133.9375 72.959) (end 133.9375 72.539002) (width 0.5) (layer F.Cu) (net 2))
 (via (at 133.9375 72.959) (size 0.5) (drill 0.3) (layers F.Cu B.Cu) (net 2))
 (via (at 132.2 75.4) (size 0.8) (drill 0.4) (layers F.Cu B.Cu) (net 10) (status 30))
 (via (at 133.33 93.67) (size 0.8) (drill 0.4) (layers F.Cu B.Cu) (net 10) (status 30))
 (via (at 134.36 93.36) (size 0.5) (drill 0.3) (layers F.Cu B.Cu) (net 10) (status 30))
 (via (at 134.39 93.97) (size 0.5) (drill 0.3) (layers F.Cu B.Cu) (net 10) (status 30))
 (segment (start 118.400001 67.440001) (end 118.400001 74.800001) (width 0.5) (layer B.Cu) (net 10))
 (segment (start 117.2 66.24) (end 118.400001 67.440001) (width 0.5) (layer B.Cu) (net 10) (status 10))
 (segment (start 118.400001 74.800001) (end 118.7 75.1) (width 0.5) (layer B.Cu) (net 10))
 (via (at 118.7 75.1) (size 0.8) (drill 0.4) (layers F.Cu B.Cu) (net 10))
 (segment (start 131.58 93.67) (end 133.33 93.67) (width 0.5) (layer F.Cu) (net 10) (status 20))
 (segment (start 119.720001 81.810001) (end 131.58 93.67) (width 0.5) (layer F.Cu) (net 10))
 (segment (start 119.720001 78.879999) (end 119.720001 81.810001) (width 0.5) (layer F.Cu) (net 10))
 (segment (start 118.7 77.859998) (end 119.720001 78.879999) (width 0.5) (layer F.Cu) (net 10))
 (segment (start 118.7 75.1) (end 118.7 77.859998) (width 0.5) (layer F.Cu) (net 10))
 (segment (start 131.834811 80.244813) (end 131.834811 92.174811) (width 0.5) (layer B.Cu) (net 10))
 (segment (start 131.749999 80.160001) (end 131.834811 80.244813) (width 0.5) (layer B.Cu) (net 10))
 (segment (start 131.834811 92.174811) (end 133.33 93.67) (width 0.5) (layer B.Cu) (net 10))
 (segment (start 131.749999 75.850001) (end 131.749999 80.160001) (width 0.5) (layer B.Cu) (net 10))
 (segment (start 132.2 75.4) (end 131.749999 75.850001) (width 0.5) (layer B.Cu) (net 10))
 (via (at 118.1 79.7) (size 0.8) (drill 0.4) (layers F.Cu B.Cu) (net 18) (status 30))
 (segment (start 115.999999 77.599999) (end 118.1 79.7) (width 0.5) (layer B.Cu) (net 18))
 (segment (start 117.2 71.32) (end 115.999999 72.520001) (width 0.5) (layer B.Cu) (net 18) (status 10))
 (segment (start 115.999999 72.520001) (end 115.999999 77.599999) (width 0.5) (layer B.Cu) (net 18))
 (segment (start 117.739998 81.66) (end 118.12 81.66) (width 0.5) (layer F.Cu) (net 17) (status 30))
 (segment (start 115.999999 79.920001) (end 117.739998 81.66) (width 0.5) (layer F.Cu) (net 17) (status 20))
 (segment (start 115.999999 69.980001) (end 115.999999 79.920001) (width 0.5) (layer F.Cu) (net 17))
 (segment (start 117.2 68.78) (end 115.999999 69.980001) (width 0.5) (layer F.Cu) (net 17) (status 10))
 (segment (start 133.4 89.7) (end 133.3 89.8) (width 0.5) (layer B.Cu) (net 16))
 (via (at 133.4 89.7) (size 0.8) (drill 0.4) (layers F.Cu B.Cu) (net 16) (status 30))
 (segment (start 135.07 89.66) (end 133.32 89.66) (width 0.5) (layer F.Cu) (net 16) (status 20))
 (segment (start 135.23599 89.49401) (end 135.07 89.66) (width 0.5) (layer F.Cu) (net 16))
 (segment (start 135.23599 83.76125) (end 135.23599 89.49401) (width 0.5) (layer F.Cu) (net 16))
 (segment (start 135.65632 83.34092) (end 135.23599 83.76125) (width 0.5) (layer F.Cu) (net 16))
 (segment (start 127.7874 77.0926) (end 126.72 78.16) (width 0.5) (layer F.Cu) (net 15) (status 20))
 (segment (start 127.7874 75.3488) (end 127.7874 77.0926) (width 0.5) (layer F.Cu) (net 15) (status 10))
 (segment (start 125.5268 75.368) (end 124.72 76.1748) (width 0.5) (layer F.Cu) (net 14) (status 10))
 (segment (start 124.72 76.1748) (end 124.72 78.16) (width 0.5) (layer F.Cu) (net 14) (status 20))
 (segment (start 125.5268 75.368) (end 125.5268 75.0443) (width 0.25) (layer F.Cu) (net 14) (status 30))
 (segment (start 120.446201 74.443799) (end 120.396 74.494) (width 0.25) (layer F.Cu) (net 14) (status 30))
 (segment (start 124.926299 74.443799) (end 120.446201 74.443799) (width 0.25) (layer F.Cu) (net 14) (status 20))
 (segment (start 125.5268 75.0443) (end 124.926299 74.443799) (width 0.25) (layer F.Cu) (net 14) (status 10))
 (via (at 131.6 64.6) (size 0.8) (drill 0.4) (layers F.Cu B.Cu) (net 9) (status 30))
 (segment (start 123 62) (end 125.7 62) (width 0.5) (layer F.Cu) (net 9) (status 10))
 (segment (start 125.7 62) (end 129.5 62) (width 0.5) (layer F.Cu) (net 9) (status 20))
 (via (at 125.7 62) (size 0.8) (drill 0.4) (layers F.Cu B.Cu) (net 9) (status 30))
 (segment (start 132.55 66.5) (end 131.2 65.15) (width 0.5) (layer B.Cu) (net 9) (status 30))
 (segment (start 133.4 66.5) (end 132.55 66.5) (width 0.5) (layer B.Cu) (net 9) (status 30))
 (segment (start 129.5 63.45) (end 129.5 62) (width 0.5) (layer B.Cu) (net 9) (status 20))
 (segment (start 131.2 65.15) (end 129.5 63.45) (width 0.5) (layer B.Cu) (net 9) (status 10))
 (segment (start 119.300001 63.899999) (end 119.169999 63.899999) (width 0.5) (layer F.Cu) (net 9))
 (via (at 119.300001 63.899999) (size 0.8) (drill 0.4) (layers F.Cu B.Cu) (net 9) (status 30))
 (segment (start 123 63.415) (end 122.4075 64.0075) (width 0.5) (layer B.Cu) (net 9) (status 20))
 (segment (start 123 62) (end 123 63.415) (width 0.5) (layer B.Cu) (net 9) (status 10))
 (segment (start 122.4075 64.0075) (end 122.385 64.03) (width 0.5) (layer B.Cu) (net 9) (status 30))
 (segment (start 119.407502 64.0075) (end 119.300001 63.899999) (width 0.5) (layer F.Cu) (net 9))
 (segment (start 122.4075 64.0075) (end 122.365 64.0075) (width 0.5) (layer F.Cu) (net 9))
 (segment (start 122.365 64.0075) (end 119.407502 64.0075) (width 0.5) (layer F.Cu) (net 9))
 (via (at 122.365 64.0075) (size 0.5) (drill 0.3) (layers F.Cu B.Cu) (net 9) (status 30))
 (segment (start 130.048 76.832) (end 128.72 78.16) (width 0.5) (layer F.Cu) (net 13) (status 20))
 (segment (start 130.048 75.3488) (end 130.048 76.832) (width 0.5) (layer F.Cu) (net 13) (status 10))
 (via (at 120.2 67.2) (size 0.8) (drill 0.4) (layers F.Cu B.Cu) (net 6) (status 30))
 (segment (start 126.057603 73.993801) (end 122.393801 73.993801) (width 0.25) (layer F.Cu) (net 7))
 (segment (start 126.501801 74.437999) (end 126.057603 73.993801) (width 0.25) (layer F.Cu) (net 7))
 (segment (start 126.501801 76.298001) (end 126.501801 74.437999) (width 0.25) (layer F.Cu) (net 7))
 (segment (start 125.994999 78.690003) (end 125.994999 76.804803) (width 0.25) (layer F.Cu) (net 7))
 (segment (start 125.400001 79.285001) (end 125.994999 78.690003) (width 0.25) (layer F.Cu) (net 7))
 (segment (start 123.845001 79.285001) (end 125.400001 79.285001) (width 0.25) (layer F.Cu) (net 7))
 (segment (start 122.72 78.16) (end 123.845001 79.285001) (width 0.25) (layer F.Cu) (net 7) (status 10))
 (segment (start 125.994999 76.804803) (end 126.501801 76.298001) (width 0.25) (layer F.Cu) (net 7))
 (segment (start 122.393801 73.993801) (end 122.2 73.8) (width 0.25) (layer F.Cu) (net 7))
 (segment (start 122.2 73.8) (end 122.2 70.3) (width 0.25) (layer F.Cu) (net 7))
 (via (at 122.2 70.3) (size 0.8) (drill 0.4) (layers F.Cu B.Cu) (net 7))
 (segment (start 122.2 68.15) (end 122.021 67.971) (width 0.25) (layer B.Cu) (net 7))
 (segment (start 122.2 70.3) (end 122.2 68.15) (width 0.25) (layer B.Cu) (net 7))
 (segment (start 122.021 67.971) (end 121.15 67.1) (width 0.25) (layer B.Cu) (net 7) (status 20))
 (via (at 122.021 67.971) (size 0.5) (drill 0.3) (layers F.Cu B.Cu) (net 7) (status 30))
 (segment (start 126.492 69.9268) (end 123.4 73.0188) (width 0.5) (layer F.Cu) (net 1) (status 20))
 (segment (start 126.492 69.088) (end 126.492 69.9268) (width 0.5) (layer F.Cu) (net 1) (status 10))
 (segment (start 123.4 75.48) (end 120.72 78.16) (width 0.5) (layer F.Cu) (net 11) (status 30))
 (segment (start 123.4 75.4188) (end 123.4 75.48) (width 0.5) (layer F.Cu) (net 11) (status 30))
 (via (at 117.8 62.5) (size 0.8) (drill 0.4) (layers F.Cu B.Cu) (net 12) (status 30))
 (segment (start 123 66.5) (end 129.5 66.5) (width 0.5) (layer F.Cu) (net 8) (status 30))
 (segment (start 120.5 72.6) (end 121.7 72.6) (width 0.5) (layer B.Cu) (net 8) (status 10))
 (segment (start 123 71.3) (end 123 66.5) (width 0.5) (layer B.Cu) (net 8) (status 20))
 (segment (start 121.7 72.6) (end 123 71.3) (width 0.5) (layer B.Cu) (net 8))
 (segment (start 121.15 63.45) (end 121.15 64.5) (width 0.5) (layer B.Cu) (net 8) (status 20))
 (segment (start 120.3 62.6) (end 121.15 63.45) (width 0.5) (layer B.Cu) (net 8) (status 10))
 (segment (start 121.15 64.65) (end 123 66.5) (width 0.5) (layer B.Cu) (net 8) (status 30))
 (segment (start 121.15 64.5) (end 121.15 64.65) (width 0.5) (layer B.Cu) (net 8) (status 30))
 (segment (start 120.550001 65.149999) (end 126.050001 65.149999) (width 0.5) (layer F.Cu) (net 4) (status 10))
 (segment (start 120.3 65.4) (end 120.550001 65.149999) (width 0.5) (layer F.Cu) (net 4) (status 30))
 (segment (start 126.050001 65.149999) (end 127.55 63.65) (width 0.5) (layer F.Cu) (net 4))
 (segment (start 127.55 63.65) (end 127.6 63.6) (width 0.5) (layer F.Cu) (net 4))
 (via (at 127.55 63.65) (size 0.8) (drill 0.4) (layers F.Cu B.Cu) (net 4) (status 30))
 (segment (start 127.65001 63.54999) (end 127.55 63.65) (width 0.5) (layer F.Cu) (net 4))
 (segment (start 134.62501 64.106493) (end 134.068507 63.54999) (width 0.5) (layer F.Cu) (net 4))
 (segment (start 134.62501 70.37149) (end 134.62501 64.106493) (width 0.5) (layer F.Cu) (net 4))
 (segment (start 134.068507 63.54999) (end 127.65001 63.54999) (width 0.5) (layer F.Cu) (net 4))
 (segment (start 133.9375 71.059) (end 134.62501 70.37149) (width 0.5) (layer F.Cu) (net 4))
 (segment (start 131.595802 78.16) (end 130.72 78.16) (width 0.5) (layer F.Cu) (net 3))
 (segment (start 133.357801 76.398001) (end 131.595802 78.16) (width 0.5) (layer F.Cu) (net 3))
 (segment (start 133.357801 75.063197) (end 133.357801 76.398001) (width 0.5) (layer F.Cu) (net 3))
 (segment (start 135.9375 72.483498) (end 133.357801 75.063197) (width 0.5) (layer F.Cu) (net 3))
 (segment (start 135.9375 72.009) (end 135.9375 72.483498) (width 0.5) (layer F.Cu) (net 3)))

